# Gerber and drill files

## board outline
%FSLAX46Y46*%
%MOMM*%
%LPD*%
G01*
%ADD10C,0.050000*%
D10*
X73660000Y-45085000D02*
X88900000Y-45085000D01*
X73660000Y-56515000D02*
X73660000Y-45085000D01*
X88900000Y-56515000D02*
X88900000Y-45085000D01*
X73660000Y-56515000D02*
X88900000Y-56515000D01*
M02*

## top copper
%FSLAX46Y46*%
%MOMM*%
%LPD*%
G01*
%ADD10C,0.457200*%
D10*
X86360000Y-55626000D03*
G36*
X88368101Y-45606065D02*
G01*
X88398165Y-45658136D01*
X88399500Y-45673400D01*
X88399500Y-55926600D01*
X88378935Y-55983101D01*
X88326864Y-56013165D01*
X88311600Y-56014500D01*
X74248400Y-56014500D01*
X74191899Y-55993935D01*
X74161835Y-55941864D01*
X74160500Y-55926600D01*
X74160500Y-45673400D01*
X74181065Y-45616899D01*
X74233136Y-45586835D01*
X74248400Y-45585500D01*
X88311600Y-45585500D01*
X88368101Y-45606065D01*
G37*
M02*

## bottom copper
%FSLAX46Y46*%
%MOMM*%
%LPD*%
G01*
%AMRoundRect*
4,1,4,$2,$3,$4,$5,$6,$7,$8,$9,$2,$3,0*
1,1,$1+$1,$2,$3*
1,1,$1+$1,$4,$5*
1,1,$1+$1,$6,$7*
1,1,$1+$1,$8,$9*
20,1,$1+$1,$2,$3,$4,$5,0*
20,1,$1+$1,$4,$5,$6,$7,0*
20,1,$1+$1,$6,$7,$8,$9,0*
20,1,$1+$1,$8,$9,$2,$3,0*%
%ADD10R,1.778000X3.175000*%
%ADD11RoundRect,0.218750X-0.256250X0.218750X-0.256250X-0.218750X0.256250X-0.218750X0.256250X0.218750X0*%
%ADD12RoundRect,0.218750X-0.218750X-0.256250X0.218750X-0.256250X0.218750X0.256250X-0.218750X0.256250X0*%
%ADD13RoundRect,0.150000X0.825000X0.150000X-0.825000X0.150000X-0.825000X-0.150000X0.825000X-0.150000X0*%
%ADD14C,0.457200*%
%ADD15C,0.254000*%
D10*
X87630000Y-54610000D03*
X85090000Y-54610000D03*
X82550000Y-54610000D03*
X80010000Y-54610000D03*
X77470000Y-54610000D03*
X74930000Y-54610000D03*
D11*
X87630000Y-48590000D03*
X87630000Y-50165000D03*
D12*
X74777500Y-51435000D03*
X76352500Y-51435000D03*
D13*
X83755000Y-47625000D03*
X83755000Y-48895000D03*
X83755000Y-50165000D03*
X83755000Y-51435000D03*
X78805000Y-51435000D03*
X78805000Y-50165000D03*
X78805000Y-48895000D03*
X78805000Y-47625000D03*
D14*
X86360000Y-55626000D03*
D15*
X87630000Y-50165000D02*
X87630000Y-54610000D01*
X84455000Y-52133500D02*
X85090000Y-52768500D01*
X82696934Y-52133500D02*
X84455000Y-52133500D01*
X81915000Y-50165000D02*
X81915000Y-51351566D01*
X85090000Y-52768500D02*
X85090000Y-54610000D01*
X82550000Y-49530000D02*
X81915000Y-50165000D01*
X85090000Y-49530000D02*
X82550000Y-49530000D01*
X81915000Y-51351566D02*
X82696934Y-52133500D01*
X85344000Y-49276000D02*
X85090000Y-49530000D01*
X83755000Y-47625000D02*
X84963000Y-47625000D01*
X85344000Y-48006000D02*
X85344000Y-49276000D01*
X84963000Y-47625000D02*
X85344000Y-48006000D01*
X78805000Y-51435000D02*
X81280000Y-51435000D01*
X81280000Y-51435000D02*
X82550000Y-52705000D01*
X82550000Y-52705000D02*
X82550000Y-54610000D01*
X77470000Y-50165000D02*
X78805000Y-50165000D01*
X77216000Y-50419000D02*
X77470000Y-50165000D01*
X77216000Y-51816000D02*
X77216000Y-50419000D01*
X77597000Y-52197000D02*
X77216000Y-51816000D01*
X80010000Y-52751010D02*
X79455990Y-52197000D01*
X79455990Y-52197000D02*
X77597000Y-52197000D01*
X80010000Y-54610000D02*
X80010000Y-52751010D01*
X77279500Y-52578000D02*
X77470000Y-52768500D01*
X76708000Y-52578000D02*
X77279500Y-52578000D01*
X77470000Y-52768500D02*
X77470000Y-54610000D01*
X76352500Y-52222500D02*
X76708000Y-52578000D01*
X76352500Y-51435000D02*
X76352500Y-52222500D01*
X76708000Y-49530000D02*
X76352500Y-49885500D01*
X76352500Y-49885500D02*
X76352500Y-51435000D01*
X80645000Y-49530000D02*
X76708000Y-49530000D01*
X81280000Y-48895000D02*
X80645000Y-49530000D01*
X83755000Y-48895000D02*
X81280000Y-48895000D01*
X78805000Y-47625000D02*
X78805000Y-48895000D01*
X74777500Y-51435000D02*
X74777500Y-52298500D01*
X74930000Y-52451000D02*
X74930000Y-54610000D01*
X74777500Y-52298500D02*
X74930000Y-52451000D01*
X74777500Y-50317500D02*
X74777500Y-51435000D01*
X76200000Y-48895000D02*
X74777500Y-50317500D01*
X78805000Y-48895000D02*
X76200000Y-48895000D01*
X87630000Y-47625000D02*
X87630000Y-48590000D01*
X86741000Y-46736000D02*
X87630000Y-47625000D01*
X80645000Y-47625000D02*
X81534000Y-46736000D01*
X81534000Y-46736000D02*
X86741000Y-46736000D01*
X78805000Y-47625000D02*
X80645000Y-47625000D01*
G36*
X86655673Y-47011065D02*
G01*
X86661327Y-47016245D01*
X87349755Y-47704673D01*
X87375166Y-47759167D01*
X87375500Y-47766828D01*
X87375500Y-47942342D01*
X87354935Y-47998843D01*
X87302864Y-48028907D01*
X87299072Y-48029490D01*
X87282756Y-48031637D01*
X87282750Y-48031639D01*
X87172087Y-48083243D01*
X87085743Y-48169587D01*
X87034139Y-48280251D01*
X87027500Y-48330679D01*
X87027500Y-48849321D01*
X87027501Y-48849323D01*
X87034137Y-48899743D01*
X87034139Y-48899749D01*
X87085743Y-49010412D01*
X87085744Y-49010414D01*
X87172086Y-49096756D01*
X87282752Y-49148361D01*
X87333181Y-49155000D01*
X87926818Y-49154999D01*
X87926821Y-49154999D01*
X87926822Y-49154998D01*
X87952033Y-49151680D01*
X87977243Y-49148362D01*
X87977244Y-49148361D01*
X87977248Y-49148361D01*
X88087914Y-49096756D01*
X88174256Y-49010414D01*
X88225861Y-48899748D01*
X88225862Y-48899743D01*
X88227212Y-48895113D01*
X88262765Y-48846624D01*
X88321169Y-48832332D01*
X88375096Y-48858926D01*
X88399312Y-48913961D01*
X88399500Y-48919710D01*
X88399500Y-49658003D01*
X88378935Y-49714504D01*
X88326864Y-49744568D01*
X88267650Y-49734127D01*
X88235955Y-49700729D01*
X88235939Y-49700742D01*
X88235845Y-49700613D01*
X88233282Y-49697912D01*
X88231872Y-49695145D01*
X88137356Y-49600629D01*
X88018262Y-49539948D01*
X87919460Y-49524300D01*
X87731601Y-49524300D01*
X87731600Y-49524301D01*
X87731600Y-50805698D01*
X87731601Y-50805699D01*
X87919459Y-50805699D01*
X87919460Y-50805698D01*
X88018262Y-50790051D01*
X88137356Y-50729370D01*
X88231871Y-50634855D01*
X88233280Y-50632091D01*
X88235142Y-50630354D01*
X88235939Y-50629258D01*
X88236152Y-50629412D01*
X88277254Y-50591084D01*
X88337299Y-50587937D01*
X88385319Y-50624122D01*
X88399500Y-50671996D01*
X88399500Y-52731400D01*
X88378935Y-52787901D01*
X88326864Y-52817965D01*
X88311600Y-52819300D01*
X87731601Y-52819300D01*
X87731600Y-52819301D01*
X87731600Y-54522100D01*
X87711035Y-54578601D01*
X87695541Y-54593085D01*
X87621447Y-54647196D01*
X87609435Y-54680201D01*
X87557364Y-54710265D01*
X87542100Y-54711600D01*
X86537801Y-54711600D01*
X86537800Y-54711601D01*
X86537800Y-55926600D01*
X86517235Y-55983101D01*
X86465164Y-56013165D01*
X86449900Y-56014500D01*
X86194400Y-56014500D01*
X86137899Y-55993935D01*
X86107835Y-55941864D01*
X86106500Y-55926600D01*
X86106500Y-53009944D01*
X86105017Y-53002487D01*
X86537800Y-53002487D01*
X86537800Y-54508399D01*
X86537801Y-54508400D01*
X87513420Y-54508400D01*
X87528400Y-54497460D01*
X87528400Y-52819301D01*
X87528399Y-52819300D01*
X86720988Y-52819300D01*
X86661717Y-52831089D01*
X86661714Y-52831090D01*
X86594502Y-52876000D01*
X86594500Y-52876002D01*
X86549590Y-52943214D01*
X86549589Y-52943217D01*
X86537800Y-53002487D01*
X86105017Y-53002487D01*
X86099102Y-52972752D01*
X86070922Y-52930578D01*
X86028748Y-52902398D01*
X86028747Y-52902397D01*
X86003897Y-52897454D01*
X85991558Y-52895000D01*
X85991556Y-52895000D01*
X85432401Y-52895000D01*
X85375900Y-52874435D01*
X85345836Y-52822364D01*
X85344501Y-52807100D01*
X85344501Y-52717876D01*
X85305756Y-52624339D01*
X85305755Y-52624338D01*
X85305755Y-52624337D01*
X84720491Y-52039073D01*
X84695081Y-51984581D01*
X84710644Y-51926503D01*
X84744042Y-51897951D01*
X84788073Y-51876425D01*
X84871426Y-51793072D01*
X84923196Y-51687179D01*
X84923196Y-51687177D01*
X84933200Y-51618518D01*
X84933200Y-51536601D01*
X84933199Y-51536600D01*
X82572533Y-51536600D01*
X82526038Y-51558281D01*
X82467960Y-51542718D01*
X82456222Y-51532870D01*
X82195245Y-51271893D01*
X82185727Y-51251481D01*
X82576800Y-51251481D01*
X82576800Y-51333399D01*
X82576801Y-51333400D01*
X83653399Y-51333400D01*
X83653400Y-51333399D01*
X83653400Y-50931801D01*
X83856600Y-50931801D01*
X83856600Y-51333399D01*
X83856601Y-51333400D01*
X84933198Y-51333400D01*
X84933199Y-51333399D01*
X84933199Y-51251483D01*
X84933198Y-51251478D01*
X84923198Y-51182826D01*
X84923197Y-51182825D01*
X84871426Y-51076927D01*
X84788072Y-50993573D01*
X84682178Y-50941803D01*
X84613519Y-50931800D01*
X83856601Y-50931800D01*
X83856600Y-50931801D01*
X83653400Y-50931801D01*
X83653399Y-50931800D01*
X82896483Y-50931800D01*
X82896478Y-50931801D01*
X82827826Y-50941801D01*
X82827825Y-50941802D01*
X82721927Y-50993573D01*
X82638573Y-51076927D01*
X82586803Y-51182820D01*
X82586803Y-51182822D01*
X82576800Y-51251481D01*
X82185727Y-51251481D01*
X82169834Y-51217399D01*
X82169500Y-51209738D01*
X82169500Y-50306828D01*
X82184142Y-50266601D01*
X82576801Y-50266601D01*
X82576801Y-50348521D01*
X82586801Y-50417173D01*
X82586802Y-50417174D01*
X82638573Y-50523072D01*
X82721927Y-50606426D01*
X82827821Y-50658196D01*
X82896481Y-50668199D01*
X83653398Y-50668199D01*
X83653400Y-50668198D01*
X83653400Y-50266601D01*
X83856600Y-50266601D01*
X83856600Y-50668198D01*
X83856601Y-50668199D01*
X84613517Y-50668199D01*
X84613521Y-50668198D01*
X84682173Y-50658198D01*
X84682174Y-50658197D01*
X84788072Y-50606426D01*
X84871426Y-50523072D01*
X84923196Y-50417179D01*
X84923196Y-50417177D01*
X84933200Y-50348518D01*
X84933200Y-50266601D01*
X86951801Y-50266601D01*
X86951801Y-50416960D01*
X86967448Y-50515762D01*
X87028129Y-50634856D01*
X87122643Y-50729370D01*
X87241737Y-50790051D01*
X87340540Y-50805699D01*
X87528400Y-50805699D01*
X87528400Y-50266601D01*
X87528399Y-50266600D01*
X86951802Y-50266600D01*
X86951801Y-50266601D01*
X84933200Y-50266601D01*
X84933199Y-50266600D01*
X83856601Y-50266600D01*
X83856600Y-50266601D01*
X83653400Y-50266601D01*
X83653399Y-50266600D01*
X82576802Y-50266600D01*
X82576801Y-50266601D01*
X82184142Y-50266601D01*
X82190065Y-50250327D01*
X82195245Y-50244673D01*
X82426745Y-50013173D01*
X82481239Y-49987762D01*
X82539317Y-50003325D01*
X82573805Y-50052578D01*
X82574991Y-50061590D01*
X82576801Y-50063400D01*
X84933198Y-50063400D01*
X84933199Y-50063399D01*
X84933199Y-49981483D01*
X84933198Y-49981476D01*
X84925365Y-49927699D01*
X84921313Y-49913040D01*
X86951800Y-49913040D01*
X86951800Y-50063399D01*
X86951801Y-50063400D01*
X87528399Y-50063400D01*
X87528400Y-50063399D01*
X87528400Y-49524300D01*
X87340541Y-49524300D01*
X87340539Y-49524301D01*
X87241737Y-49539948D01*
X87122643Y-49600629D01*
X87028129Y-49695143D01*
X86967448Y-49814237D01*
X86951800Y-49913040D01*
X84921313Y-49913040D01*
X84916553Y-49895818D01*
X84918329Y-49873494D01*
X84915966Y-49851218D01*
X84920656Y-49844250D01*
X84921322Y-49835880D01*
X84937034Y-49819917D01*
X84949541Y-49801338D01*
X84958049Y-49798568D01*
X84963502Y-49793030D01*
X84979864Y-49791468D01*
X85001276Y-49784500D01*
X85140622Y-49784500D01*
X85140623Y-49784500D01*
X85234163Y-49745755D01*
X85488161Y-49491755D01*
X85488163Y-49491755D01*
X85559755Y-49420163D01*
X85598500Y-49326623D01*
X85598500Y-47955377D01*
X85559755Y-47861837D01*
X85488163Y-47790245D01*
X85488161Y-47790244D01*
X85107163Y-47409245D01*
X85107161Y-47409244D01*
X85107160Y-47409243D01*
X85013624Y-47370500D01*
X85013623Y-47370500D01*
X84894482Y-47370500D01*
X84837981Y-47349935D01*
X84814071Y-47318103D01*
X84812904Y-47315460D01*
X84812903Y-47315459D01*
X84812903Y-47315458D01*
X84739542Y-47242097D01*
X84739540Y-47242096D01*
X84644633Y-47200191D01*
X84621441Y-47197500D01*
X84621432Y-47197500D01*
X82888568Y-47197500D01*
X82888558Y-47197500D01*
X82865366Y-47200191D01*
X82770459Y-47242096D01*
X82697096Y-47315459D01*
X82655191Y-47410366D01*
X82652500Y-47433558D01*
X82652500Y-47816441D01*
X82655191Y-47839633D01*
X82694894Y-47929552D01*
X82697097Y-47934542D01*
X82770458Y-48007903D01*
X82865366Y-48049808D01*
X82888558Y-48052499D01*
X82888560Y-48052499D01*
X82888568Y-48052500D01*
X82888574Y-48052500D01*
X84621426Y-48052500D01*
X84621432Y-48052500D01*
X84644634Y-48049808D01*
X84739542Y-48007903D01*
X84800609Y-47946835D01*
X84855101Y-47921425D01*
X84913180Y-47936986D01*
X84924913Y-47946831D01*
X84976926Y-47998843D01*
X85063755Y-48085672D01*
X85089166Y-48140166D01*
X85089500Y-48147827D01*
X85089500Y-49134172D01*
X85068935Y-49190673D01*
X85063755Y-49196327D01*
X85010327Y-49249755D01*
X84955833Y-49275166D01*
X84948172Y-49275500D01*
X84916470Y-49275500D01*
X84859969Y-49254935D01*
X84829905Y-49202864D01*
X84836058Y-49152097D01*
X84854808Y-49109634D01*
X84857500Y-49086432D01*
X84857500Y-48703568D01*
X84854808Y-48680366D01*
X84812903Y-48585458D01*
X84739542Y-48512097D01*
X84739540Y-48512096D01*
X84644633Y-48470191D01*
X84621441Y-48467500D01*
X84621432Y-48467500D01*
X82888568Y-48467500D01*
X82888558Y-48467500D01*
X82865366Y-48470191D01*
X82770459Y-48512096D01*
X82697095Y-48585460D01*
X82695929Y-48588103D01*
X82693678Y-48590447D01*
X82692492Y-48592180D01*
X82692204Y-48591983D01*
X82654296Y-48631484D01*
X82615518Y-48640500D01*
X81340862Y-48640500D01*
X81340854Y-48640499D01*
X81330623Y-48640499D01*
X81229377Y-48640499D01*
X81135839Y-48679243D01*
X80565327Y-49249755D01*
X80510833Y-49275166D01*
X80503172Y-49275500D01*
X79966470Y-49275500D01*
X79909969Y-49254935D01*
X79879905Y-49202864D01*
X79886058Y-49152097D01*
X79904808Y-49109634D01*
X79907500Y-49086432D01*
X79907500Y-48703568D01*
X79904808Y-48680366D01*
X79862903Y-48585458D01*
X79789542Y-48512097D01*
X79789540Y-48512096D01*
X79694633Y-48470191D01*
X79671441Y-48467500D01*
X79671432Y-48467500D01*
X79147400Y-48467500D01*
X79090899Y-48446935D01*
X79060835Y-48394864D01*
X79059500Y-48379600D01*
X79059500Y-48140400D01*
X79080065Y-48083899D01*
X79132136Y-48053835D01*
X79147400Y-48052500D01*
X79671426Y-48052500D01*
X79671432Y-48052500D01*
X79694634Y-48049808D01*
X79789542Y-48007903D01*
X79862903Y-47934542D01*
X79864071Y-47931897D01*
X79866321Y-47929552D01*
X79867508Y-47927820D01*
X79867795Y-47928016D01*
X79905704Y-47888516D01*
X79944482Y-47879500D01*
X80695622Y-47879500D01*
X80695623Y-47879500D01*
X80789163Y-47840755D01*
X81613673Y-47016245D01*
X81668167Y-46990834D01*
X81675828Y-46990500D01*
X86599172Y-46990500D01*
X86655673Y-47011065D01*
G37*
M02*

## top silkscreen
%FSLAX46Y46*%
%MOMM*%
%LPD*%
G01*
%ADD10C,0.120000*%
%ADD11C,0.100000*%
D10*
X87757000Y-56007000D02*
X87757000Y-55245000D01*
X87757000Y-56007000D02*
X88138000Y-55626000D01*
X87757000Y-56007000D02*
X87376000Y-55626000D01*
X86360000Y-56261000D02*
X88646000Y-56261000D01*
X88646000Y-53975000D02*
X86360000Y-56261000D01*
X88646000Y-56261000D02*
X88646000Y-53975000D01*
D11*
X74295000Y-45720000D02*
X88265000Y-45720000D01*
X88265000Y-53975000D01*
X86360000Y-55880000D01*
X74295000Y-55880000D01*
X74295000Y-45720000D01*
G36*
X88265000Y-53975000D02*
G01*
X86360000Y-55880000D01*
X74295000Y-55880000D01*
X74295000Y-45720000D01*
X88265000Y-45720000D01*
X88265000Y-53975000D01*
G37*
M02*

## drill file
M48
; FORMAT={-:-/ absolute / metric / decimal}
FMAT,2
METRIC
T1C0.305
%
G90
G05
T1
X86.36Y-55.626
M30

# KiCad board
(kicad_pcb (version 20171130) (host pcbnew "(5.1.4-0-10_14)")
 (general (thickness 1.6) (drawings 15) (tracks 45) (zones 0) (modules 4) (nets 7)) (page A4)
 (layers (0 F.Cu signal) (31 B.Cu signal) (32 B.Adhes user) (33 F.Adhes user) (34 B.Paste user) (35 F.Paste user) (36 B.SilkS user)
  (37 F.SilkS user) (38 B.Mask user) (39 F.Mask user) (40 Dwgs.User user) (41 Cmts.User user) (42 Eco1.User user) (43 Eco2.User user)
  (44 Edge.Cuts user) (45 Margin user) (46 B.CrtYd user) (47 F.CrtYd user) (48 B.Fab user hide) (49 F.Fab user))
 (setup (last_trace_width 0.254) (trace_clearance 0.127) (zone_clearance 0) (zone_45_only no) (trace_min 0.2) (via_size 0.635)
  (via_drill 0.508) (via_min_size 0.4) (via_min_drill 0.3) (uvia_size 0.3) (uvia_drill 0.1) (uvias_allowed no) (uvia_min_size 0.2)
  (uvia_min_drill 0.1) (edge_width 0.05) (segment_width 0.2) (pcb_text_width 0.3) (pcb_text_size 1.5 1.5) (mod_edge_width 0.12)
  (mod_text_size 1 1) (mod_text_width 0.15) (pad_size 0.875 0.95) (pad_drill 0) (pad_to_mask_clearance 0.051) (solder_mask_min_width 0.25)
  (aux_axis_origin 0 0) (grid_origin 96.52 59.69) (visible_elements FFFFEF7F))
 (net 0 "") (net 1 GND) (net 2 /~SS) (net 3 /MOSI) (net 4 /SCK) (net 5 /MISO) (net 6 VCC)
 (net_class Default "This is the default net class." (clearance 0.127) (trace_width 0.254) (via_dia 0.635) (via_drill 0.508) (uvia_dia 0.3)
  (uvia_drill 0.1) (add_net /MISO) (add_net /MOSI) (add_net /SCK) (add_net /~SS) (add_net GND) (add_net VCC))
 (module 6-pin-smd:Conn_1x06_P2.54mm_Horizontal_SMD (layer B.Cu) (at 81.28 50.8 180)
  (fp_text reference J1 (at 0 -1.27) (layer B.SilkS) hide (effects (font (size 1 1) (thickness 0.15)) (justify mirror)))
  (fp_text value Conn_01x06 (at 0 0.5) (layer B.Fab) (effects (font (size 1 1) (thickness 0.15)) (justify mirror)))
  (pad 1 smd rect (at -6.35 -3.81 180) (size 1.778 3.175) (layers B.Cu B.Paste B.Mask) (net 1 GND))
  (pad 2 smd rect (at -3.81 -3.81 180) (size 1.778 3.175) (layers B.Cu B.Paste B.Mask) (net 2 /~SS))
  (pad 3 smd rect (at -1.27 -3.81 180) (size 1.778 3.175) (layers B.Cu B.Paste B.Mask) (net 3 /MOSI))
  (pad 4 smd rect (at 1.27 -3.81 180) (size 1.778 3.175) (layers B.Cu B.Paste B.Mask) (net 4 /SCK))
  (pad 5 smd rect (at 3.81 -3.81 180) (size 1.778 3.175) (layers B.Cu B.Paste B.Mask) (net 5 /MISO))
  (pad 6 smd rect (at 6.35 -3.81 180) (size 1.778 3.175) (layers B.Cu B.Paste B.Mask) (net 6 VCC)))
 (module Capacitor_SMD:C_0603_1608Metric (layer B.Cu) (at 87.63 49.3775 270)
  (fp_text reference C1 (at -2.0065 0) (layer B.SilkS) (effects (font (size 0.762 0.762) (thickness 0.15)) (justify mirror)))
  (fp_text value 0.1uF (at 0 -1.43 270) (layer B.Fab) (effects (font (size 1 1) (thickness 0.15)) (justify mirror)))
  (pad 1 smd roundrect (at -0.7875 0 270) (size 0.875 0.95) (layers B.Cu B.Paste B.Mask) (roundrect_rratio 0.25) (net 6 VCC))
  (pad 2 smd roundrect (at 0.7875 0 270) (size 0.875 0.95) (layers B.Cu B.Paste B.Mask) (roundrect_rratio 0.25) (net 1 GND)))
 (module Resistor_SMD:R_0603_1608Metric (layer B.Cu) (at 75.565 51.435)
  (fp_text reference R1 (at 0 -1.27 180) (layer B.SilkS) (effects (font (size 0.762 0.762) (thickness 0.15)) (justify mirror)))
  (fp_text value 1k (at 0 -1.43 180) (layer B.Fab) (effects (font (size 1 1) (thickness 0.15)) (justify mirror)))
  (pad 1 smd roundrect (at -0.7875 0) (size 0.875 0.95) (layers B.Cu B.Paste B.Mask) (roundrect_rratio 0.25) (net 6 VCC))
  (pad 2 smd roundrect (at 0.7875 0) (size 0.875 0.95) (layers B.Cu B.Paste B.Mask) (roundrect_rratio 0.25) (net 5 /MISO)))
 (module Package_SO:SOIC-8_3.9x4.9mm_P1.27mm (layer B.Cu) (at 81.28 49.53 180)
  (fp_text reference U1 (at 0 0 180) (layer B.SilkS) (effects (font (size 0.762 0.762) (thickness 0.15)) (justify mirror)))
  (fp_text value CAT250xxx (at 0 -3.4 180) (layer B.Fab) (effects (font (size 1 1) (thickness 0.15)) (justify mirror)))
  (pad 1 smd roundrect (at -2.475 1.905 180) (size 1.95 0.6) (layers B.Cu B.Paste B.Mask) (roundrect_rratio 0.25) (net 2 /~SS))
  (pad 2 smd roundrect (at -2.475 0.635 180) (size 1.95 0.6) (layers B.Cu B.Paste B.Mask) (roundrect_rratio 0.25) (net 5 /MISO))
  (pad 3 smd roundrect (at -2.475 -0.635 180) (size 1.95 0.6) (layers B.Cu B.Paste B.Mask) (roundrect_rratio 0.25) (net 1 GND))
  (pad 4 smd roundrect (at -2.475 -1.905 180) (size 1.95 0.6) (layers B.Cu B.Paste B.Mask) (roundrect_rratio 0.25) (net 1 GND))
  (pad 5 smd roundrect (at 2.475 -1.905 180) (size 1.95 0.6) (layers B.Cu B.Paste B.Mask) (roundrect_rratio 0.25) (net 3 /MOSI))
  (pad 6 smd roundrect (at 2.475 -0.635 180) (size 1.95 0.6) (layers B.Cu B.Paste B.Mask) (roundrect_rratio 0.25) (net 4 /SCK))
  (pad 7 smd roundrect (at 2.475 0.635 180) (size 1.95 0.6) (layers B.Cu B.Paste B.Mask) (roundrect_rratio 0.25) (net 6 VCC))
  (pad 8 smd roundrect (at 2.475 1.905 180) (size 1.95 0.6) (layers B.Cu B.Paste B.Mask) (roundrect_rratio 0.25) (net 6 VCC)))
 (gr_line (start 87.757 56.007) (end 87.757 55.245) (layer F.SilkS) (width 0.12))
 (gr_line (start 87.757 56.007) (end 88.138 55.626) (layer F.SilkS) (width 0.12))
 (gr_line (start 87.757 56.007) (end 87.376 55.626) (layer F.SilkS) (width 0.12))
 (gr_line (start 86.36 56.261) (end 88.646 56.261) (layer F.SilkS) (width 0.12))
 (gr_line (start 88.646 53.975) (end 86.36 56.261) (layer F.SilkS) (width 0.12))
 (gr_line (start 88.646 56.261) (end 88.646 53.975) (layer F.SilkS) (width 0.12))
 (gr_poly (pts (xy 74.295 45.72) (xy 88.265 45.72) (xy 88.265 53.975) (xy 86.36 55.88) (xy 74.295 55.88)) (layer F.SilkS) (width 0.1))
 (gr_line (start 73.66 45.085) (end 88.9 45.085) (layer Edge.Cuts) (width 0.05))
 (gr_line (start 73.66 56.515) (end 73.66 45.085) (layer Edge.Cuts) (width 0.05))
 (gr_line (start 88.9 56.515) (end 88.9 45.085) (layer Edge.Cuts) (width 0.05))
 (gr_line (start 73.66 56.515) (end 88.9 56.515) (layer Edge.Cuts) (width 0.05))
 (via (at 86.36 55.626) (size 0.4572) (drill 0.3048) (layers F.Cu B.Cu) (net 1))
 (segment (start 87.63 50.165) (end 87.63 54.61) (width 0.254) (layer B.Cu) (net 1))
 (segment (start 84.455 52.1335) (end 85.09 52.7685) (width 0.254) (layer B.Cu) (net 2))
 (segment (start 82.696934 52.1335) (end 84.455 52.1335) (width 0.254) (layer B.Cu) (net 2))
 (segment (start 81.915 50.165) (end 81.915 51.351566) (width 0.254) (layer B.Cu) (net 2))
 (segment (start 85.09 52.7685) (end 85.09 54.61) (width 0.254) (layer B.Cu) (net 2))
 (segment (start 82.55 49.53) (end 81.915 50.165) (width 0.254) (layer B.Cu) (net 2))
 (segment (start 85.09 49.53) (end 82.55 49.53) (width 0.254) (layer B.Cu) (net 2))
 (segment (start 81.915 51.351566) (end 82.696934 52.1335) (width 0.254) (layer B.Cu) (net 2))
 (segment (start 85.344 49.276) (end 85.09 49.53) (width 0.254) (layer B.Cu) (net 2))
 (segment (start 83.755 47.625) (end 84.963 47.625) (width 0.254) (layer B.Cu) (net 2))
 (segment (start 85.344 48.006) (end 85.344 49.276) (width 0.254) (layer B.Cu) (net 2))
 (segment (start 84.963 47.625) (end 85.344 48.006) (width 0.254) (layer B.Cu) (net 2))
 (segment (start 78.805 51.435) (end 81.28 51.435) (width 0.254) (layer B.Cu) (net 3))
 (segment (start 81.28 51.435) (end 82.55 52.705) (width 0.254) (layer B.Cu) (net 3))
 (segment (start 82.55 52.705) (end 82.55 54.61) (width 0.254) (layer B.Cu) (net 3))
 (segment (start 77.47 50.165) (end 78.805 50.165) (width 0.254) (layer B.Cu) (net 4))
 (segment (start 77.216 50.419) (end 77.47 50.165) (width 0.254) (layer B.Cu) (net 4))
 (segment (start 77.216 51.816) (end 77.216 50.419) (width 0.254) (layer B.Cu) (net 4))
 (segment (start 77.597 52.197) (end 77.216 51.816) (width 0.254) (layer B.Cu) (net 4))
 (segment (start 80.01 52.75101) (end 79.45599 52.197) (width 0.254) (layer B.Cu) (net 4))
 (segment (start 79.45599 52.197) (end 77.597 52.197) (width 0.254) (layer B.Cu) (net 4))
 (segment (start 80.01 54.61) (end 80.01 52.75101) (width 0.254) (layer B.Cu) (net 4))
 (segment (start 77.2795 52.578) (end 77.47 52.7685) (width 0.254) (layer B.Cu) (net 5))
 (segment (start 76.708 52.578) (end 77.2795 52.578) (width 0.254) (layer B.Cu) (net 5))
 (segment (start 77.47 52.7685) (end 77.47 54.61) (width 0.254) (layer B.Cu) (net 5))
 (segment (start 76.3525 52.2225) (end 76.708 52.578) (width 0.254) (layer B.Cu) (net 5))
 (segment (start 76.3525 51.435) (end 76.3525 52.2225) (width 0.254) (layer B.Cu) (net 5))
 (segment (start 76.708 49.53) (end 76.3525 49.8855) (width 0.254) (layer B.Cu) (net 5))
 (segment (start 76.3525 49.8855) (end 76.3525 51.435) (width 0.254) (layer B.Cu) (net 5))
 (segment (start 80.645 49.53) (end 76.708 49.53) (width 0.254) (layer B.Cu) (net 5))
 (segment (start 81.28 48.895) (end 80.645 49.53) (width 0.254) (layer B.Cu) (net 5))
 (segment (start 83.755 48.895) (end 81.28 48.895) (width 0.254) (layer B.Cu) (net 5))
 (segment (start 78.805 47.625) (end 78.805 48.895) (width 0.254) (layer B.Cu) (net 6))
 (segment (start 74.7775 51.435) (end 74.7775 52.2985) (width 0.254) (layer B.Cu) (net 6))
 (segment (start 74.93 52.451) (end 74.93 54.61) (width 0.254) (layer B.Cu) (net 6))
 (segment (start 74.7775 52.2985) (end 74.93 52.451) (width 0.254) (layer B.Cu) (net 6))
 (segment (start 74.7775 50.3175) (end 74.7775 51.435) (width 0.254) (layer B.Cu) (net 6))
 (segment (start 76.2 48.895) (end 74.7775 50.3175) (width 0.254) (layer B.Cu) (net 6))
 (segment (start 78.805 48.895) (end 76.2 48.895) (width 0.254) (layer B.Cu) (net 6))
 (segment (start 87.63 47.625) (end 87.63 48.59) (width 0.254) (layer B.Cu) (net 6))
 (segment (start 86.741 46.736) (end 87.63 47.625) (width 0.254) (layer B.Cu) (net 6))
 (segment (start 80.645 47.625) (end 81.534 46.736) (width 0.254) (layer B.Cu) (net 6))
 (segment (start 81.534 46.736) (end 86.741 46.736) (width 0.254) (layer B.Cu) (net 6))
 (segment (start 78.805 47.625) (end 80.645 47.625) (width 0.254) (layer B.Cu) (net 6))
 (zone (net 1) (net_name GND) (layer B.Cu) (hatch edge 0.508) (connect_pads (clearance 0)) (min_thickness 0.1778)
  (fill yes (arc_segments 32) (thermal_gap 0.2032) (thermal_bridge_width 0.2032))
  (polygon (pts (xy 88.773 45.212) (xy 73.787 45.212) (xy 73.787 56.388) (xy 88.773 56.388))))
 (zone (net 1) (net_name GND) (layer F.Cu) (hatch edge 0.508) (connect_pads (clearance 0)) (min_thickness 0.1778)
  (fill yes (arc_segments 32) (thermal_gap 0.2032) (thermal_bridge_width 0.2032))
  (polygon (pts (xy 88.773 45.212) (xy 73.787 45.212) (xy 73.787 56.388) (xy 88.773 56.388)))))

